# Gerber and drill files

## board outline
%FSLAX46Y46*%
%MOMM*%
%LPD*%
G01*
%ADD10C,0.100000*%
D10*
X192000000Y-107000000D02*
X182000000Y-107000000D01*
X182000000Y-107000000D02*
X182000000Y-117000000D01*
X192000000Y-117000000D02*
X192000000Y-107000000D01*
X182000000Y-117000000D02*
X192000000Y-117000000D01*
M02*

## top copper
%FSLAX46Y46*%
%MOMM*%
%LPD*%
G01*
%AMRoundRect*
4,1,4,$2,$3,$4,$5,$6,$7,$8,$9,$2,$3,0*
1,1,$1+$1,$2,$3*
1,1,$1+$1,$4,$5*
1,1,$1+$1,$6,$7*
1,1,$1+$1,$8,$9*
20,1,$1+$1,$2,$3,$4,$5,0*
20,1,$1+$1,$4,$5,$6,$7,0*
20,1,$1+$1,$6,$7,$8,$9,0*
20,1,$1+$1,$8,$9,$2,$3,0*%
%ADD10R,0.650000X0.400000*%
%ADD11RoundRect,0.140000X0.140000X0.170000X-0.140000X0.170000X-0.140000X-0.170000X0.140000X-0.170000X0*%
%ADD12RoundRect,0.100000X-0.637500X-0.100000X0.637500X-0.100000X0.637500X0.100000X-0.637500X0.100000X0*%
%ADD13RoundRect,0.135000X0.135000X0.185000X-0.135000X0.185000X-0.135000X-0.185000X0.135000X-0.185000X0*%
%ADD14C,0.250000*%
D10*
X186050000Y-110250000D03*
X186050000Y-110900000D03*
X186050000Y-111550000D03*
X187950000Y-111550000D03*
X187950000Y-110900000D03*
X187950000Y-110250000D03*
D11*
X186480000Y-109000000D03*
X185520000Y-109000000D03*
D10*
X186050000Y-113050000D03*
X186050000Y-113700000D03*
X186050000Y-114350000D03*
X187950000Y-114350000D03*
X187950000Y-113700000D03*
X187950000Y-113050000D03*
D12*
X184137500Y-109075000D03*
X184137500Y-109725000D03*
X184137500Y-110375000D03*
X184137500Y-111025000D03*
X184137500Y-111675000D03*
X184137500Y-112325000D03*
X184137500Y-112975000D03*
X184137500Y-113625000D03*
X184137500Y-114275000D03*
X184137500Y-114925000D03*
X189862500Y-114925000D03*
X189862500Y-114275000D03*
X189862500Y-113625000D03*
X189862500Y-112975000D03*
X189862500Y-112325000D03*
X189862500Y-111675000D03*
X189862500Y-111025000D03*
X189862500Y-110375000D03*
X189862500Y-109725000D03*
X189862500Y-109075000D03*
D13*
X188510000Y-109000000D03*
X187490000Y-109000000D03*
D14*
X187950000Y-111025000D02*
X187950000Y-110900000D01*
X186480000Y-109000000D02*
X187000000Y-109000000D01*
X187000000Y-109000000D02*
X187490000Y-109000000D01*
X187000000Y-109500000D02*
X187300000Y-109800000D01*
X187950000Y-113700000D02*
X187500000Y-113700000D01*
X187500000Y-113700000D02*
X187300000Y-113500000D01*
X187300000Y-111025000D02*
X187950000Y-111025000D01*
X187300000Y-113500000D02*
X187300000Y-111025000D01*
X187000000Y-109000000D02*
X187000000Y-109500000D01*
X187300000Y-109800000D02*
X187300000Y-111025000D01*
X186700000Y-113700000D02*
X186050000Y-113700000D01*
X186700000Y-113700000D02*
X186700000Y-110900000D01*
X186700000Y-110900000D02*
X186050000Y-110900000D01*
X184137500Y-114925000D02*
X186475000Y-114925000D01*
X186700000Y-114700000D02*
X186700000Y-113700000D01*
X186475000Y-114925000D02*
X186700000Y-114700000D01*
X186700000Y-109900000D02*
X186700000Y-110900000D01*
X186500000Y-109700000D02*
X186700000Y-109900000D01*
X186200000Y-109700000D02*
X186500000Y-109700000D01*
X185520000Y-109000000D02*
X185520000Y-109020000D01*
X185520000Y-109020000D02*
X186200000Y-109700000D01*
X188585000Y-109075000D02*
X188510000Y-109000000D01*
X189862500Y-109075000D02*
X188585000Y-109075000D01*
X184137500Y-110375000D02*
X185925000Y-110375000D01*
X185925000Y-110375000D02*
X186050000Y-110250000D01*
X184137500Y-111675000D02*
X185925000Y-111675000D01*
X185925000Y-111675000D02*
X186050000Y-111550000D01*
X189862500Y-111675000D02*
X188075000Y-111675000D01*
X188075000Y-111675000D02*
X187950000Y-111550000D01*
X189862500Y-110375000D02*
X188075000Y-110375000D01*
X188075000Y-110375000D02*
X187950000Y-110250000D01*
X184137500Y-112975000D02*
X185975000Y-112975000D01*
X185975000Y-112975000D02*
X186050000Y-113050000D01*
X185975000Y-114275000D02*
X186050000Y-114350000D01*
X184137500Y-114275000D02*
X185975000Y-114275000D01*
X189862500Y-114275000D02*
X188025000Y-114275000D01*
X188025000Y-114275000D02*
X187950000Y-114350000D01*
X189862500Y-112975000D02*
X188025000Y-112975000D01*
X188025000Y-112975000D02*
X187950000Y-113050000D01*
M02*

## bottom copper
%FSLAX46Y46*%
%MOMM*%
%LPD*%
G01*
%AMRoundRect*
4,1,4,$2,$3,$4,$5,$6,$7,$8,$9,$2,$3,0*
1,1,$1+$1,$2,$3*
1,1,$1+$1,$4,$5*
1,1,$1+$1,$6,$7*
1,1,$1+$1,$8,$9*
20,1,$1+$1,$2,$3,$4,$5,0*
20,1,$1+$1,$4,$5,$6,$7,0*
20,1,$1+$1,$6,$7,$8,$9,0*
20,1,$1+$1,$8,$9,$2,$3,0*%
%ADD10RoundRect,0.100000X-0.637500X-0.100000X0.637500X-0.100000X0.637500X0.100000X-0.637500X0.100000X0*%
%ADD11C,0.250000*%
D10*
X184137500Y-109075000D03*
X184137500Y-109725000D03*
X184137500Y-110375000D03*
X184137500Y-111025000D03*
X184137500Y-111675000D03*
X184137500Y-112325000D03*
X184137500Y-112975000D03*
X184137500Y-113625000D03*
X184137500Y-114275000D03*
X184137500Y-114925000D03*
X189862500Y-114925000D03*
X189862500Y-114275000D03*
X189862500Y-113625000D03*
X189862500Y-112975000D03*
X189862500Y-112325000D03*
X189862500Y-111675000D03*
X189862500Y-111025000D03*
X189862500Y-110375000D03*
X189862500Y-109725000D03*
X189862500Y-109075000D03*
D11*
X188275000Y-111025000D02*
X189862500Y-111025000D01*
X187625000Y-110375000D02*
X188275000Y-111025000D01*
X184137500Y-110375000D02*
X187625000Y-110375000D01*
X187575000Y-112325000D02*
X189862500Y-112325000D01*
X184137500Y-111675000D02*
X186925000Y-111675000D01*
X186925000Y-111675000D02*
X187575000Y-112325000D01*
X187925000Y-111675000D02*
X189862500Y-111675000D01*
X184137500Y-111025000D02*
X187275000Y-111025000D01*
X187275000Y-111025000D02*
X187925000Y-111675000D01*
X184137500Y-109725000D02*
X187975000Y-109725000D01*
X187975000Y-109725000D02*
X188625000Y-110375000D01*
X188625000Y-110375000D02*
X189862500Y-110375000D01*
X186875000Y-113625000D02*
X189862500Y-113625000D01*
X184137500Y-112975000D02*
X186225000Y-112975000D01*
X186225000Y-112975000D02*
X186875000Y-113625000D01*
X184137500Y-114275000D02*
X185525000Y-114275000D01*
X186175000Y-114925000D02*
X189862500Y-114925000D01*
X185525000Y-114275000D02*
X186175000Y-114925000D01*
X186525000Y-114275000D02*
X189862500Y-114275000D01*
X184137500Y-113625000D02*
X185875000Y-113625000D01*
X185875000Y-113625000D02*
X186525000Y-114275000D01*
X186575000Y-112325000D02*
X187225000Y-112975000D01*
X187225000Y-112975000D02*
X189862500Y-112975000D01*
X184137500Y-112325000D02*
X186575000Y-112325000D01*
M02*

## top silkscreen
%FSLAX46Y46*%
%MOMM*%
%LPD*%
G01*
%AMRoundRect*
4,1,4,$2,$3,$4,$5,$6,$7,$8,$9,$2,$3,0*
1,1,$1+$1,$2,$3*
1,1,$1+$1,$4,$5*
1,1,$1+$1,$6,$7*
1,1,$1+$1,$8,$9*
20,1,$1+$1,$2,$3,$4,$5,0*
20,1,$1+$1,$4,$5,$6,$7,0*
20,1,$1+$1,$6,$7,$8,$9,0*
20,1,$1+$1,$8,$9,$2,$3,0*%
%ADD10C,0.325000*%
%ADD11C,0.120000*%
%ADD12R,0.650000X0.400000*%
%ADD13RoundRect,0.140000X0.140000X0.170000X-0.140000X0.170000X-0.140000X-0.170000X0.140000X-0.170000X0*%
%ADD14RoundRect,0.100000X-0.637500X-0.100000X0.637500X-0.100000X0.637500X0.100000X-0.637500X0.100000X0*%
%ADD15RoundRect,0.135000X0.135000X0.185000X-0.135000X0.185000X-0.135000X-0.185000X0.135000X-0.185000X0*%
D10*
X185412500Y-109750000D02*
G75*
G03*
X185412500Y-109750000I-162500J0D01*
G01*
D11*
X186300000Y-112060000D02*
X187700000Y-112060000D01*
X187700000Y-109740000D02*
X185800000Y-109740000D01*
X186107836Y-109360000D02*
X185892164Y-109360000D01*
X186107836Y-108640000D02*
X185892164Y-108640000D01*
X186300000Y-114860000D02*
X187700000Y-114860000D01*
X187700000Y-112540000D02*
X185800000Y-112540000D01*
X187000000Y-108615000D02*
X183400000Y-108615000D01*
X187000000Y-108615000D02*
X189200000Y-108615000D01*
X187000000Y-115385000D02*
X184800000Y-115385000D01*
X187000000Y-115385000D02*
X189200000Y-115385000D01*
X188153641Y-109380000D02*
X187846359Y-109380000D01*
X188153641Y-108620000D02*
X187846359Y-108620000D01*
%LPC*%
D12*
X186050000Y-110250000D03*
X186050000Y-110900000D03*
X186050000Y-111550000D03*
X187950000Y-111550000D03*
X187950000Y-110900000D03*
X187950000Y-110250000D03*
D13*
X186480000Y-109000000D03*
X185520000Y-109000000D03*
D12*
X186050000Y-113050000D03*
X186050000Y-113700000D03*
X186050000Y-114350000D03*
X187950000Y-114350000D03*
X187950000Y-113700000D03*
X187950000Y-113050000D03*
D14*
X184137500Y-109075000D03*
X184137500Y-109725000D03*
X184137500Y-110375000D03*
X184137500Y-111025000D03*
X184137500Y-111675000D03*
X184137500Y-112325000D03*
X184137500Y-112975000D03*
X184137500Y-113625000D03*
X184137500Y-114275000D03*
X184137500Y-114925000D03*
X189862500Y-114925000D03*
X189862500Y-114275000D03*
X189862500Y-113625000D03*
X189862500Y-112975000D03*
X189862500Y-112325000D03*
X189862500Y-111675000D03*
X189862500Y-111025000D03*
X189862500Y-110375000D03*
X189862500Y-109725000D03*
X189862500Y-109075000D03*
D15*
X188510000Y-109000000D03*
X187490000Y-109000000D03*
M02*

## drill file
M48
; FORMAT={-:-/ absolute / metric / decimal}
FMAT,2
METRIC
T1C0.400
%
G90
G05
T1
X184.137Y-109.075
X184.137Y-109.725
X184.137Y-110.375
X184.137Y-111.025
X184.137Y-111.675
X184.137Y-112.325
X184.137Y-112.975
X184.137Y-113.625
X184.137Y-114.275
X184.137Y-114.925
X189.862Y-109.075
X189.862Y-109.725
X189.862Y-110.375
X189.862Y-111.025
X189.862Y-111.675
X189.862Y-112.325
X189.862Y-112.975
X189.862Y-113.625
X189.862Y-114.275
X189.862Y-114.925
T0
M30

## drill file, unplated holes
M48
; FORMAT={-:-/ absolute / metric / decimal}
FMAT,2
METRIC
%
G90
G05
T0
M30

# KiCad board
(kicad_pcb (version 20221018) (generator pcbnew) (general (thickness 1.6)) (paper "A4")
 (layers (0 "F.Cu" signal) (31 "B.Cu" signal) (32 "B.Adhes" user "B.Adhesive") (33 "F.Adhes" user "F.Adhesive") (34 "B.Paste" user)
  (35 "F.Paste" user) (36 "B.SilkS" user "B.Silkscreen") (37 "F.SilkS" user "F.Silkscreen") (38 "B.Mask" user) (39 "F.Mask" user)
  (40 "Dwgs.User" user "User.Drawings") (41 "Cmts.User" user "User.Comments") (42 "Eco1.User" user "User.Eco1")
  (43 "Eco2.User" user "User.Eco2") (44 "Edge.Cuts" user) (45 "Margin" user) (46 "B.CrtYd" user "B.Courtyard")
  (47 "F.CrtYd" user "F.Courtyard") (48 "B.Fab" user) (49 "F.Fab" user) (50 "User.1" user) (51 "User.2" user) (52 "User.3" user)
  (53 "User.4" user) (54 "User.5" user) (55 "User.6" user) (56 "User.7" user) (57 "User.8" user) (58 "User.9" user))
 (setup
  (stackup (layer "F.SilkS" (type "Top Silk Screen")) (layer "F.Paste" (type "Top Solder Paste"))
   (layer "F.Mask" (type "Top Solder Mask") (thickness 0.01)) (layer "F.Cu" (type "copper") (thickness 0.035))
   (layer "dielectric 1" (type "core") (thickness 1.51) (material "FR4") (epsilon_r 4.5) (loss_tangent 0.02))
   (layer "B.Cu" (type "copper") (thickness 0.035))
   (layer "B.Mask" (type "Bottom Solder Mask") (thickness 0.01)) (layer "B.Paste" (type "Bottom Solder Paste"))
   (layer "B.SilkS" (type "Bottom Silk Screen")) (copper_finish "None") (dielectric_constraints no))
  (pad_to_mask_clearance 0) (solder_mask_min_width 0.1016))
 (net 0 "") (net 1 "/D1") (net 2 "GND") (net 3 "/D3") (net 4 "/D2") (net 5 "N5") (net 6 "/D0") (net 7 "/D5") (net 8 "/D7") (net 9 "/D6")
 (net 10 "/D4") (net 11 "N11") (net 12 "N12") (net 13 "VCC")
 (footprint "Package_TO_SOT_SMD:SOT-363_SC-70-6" (layer "F.Cu") (at 187 110.9)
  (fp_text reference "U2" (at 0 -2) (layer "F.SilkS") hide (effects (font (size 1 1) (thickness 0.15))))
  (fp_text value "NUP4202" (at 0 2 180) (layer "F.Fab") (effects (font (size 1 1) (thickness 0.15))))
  (fp_line (start -0.7 1.16) (end 0.7 1.16) (stroke (width 0.12) (type solid)) (layer "F.SilkS"))
  (fp_line (start 0.7 -1.16) (end -1.2 -1.16) (stroke (width 0.12) (type solid)) (layer "F.SilkS"))
  (pad "1" smd rect (at -0.95 -0.65) (size 0.65 0.4) (layers "F.Cu" "F.Paste" "F.Mask") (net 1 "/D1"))
  (pad "2" smd rect (at -0.95 0) (size 0.65 0.4) (layers "F.Cu" "F.Paste" "F.Mask") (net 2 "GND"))
  (pad "3" smd rect (at -0.95 0.65) (size 0.65 0.4) (layers "F.Cu" "F.Paste" "F.Mask") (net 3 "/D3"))
  (pad "4" smd rect (at 0.95 0.65) (size 0.65 0.4) (layers "F.Cu" "F.Paste" "F.Mask") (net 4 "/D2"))
  (pad "5" smd rect (at 0.95 0) (size 0.65 0.4) (layers "F.Cu" "F.Paste" "F.Mask") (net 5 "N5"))
  (pad "6" smd rect (at 0.95 -0.65) (size 0.65 0.4) (layers "F.Cu" "F.Paste" "F.Mask") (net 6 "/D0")))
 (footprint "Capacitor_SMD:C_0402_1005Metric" (layer "F.Cu") (at 186 109 180)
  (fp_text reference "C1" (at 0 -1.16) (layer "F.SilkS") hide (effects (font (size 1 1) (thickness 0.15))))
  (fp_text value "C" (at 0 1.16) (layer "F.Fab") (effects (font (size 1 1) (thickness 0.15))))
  (fp_line (start -0.107836 -0.36) (end 0.107836 -0.36) (stroke (width 0.12) (type solid)) (layer "F.SilkS"))
  (fp_line (start -0.107836 0.36) (end 0.107836 0.36) (stroke (width 0.12) (type solid)) (layer "F.SilkS"))
  (pad "1" smd roundrect (at -0.48 0 180) (size 0.56 0.62) (layers "F.Cu" "F.Paste" "F.Mask") (roundrect_rratio 0.25) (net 5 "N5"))
  (pad "2" smd roundrect (at 0.48 0 180) (size 0.56 0.62) (layers "F.Cu" "F.Paste" "F.Mask") (roundrect_rratio 0.25) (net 2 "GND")))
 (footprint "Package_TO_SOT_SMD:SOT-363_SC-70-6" (layer "F.Cu") (at 187 113.7)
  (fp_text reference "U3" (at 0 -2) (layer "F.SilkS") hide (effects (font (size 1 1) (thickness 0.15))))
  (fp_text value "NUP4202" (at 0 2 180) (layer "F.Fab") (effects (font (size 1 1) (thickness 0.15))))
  (fp_line (start -0.7 1.16) (end 0.7 1.16) (stroke (width 0.12) (type solid)) (layer "F.SilkS"))
  (fp_line (start 0.7 -1.16) (end -1.2 -1.16) (stroke (width 0.12) (type solid)) (layer "F.SilkS"))
  (pad "1" smd rect (at -0.95 -0.65) (size 0.65 0.4) (layers "F.Cu" "F.Paste" "F.Mask") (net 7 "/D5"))
  (pad "2" smd rect (at -0.95 0) (size 0.65 0.4) (layers "F.Cu" "F.Paste" "F.Mask") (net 2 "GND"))
  (pad "3" smd rect (at -0.95 0.65) (size 0.65 0.4) (layers "F.Cu" "F.Paste" "F.Mask") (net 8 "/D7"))
  (pad "4" smd rect (at 0.95 0.65) (size 0.65 0.4) (layers "F.Cu" "F.Paste" "F.Mask") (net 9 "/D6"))
  (pad "5" smd rect (at 0.95 0) (size 0.65 0.4) (layers "F.Cu" "F.Paste" "F.Mask") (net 5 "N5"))
  (pad "6" smd rect (at 0.95 -0.65) (size 0.65 0.4) (layers "F.Cu" "F.Paste" "F.Mask") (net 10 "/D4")))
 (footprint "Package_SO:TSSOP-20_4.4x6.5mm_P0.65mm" (layer "F.Cu") (at 187 112)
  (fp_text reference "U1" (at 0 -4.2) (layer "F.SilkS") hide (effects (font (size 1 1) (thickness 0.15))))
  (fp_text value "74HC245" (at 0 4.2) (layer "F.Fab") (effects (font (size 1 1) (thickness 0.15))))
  (fp_line (start 0 -3.385) (end -3.6 -3.385) (stroke (width 0.12) (type solid)) (layer "F.SilkS"))
  (fp_line (start 0 -3.385) (end 2.2 -3.385) (stroke (width 0.12) (type solid)) (layer "F.SilkS"))
  (fp_line (start 0 3.385) (end -2.2 3.385) (stroke (width 0.12) (type solid)) (layer "F.SilkS"))
  (fp_line (start 0 3.385) (end 2.2 3.385) (stroke (width 0.12) (type solid)) (layer "F.SilkS"))
  (pad "1" thru_hole roundrect (at -2.8625 -2.925) (size 1.475 0.4) (drill 0.4) (layers "*.Cu" "*.Mask") (roundrect_rratio 0.25)
   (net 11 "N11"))
  (pad "2" thru_hole roundrect (at -2.8625 -2.275) (size 1.475 0.4) (drill 0.4) (layers "*.Cu" "*.Mask") (roundrect_rratio 0.25)
   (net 6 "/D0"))
  (pad "3" thru_hole roundrect (at -2.8625 -1.625) (size 1.475 0.4) (drill 0.4) (layers "*.Cu" "*.Mask") (roundrect_rratio 0.25)
   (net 1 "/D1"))
  (pad "4" thru_hole roundrect (at -2.8625 -0.975) (size 1.475 0.4) (drill 0.4) (layers "*.Cu" "*.Mask") (roundrect_rratio 0.25)
   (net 4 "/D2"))
  (pad "5" thru_hole roundrect (at -2.8625 -0.325) (size 1.475 0.4) (drill 0.4) (layers "*.Cu" "*.Mask") (roundrect_rratio 0.25)
   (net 3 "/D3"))
  (pad "6" thru_hole roundrect (at -2.8625 0.325) (size 1.475 0.4) (drill 0.4) (layers "*.Cu" "*.Mask") (roundrect_rratio 0.25)
   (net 10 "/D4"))
  (pad "7" thru_hole roundrect (at -2.8625 0.975) (size 1.475 0.4) (drill 0.4) (layers "*.Cu" "*.Mask") (roundrect_rratio 0.25)
   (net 7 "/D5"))
  (pad "8" thru_hole roundrect (at -2.8625 1.625) (size 1.475 0.4) (drill 0.4) (layers "*.Cu" "*.Mask") (roundrect_rratio 0.25)
   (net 9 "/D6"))
  (pad "9" thru_hole roundrect (at -2.8625 2.275) (size 1.475 0.4) (drill 0.4) (layers "*.Cu" "*.Mask") (roundrect_rratio 0.25)
   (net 8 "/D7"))
  (pad "10" thru_hole roundrect (at -2.8625 2.925) (size 1.475 0.4) (drill 0.4) (layers "*.Cu" "*.Mask") (roundrect_rratio 0.25)
   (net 2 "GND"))
  (pad "11" thru_hole roundrect (at 2.8625 2.925) (size 1.475 0.4) (drill 0.4) (layers "*.Cu" "*.Mask") (roundrect_rratio 0.25)
   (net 8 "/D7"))
  (pad "12" thru_hole roundrect (at 2.8625 2.275) (size 1.475 0.4) (drill 0.4) (layers "*.Cu" "*.Mask") (roundrect_rratio 0.25)
   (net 9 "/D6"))
  (pad "13" thru_hole roundrect (at 2.8625 1.625) (size 1.475 0.4) (drill 0.4) (layers "*.Cu" "*.Mask") (roundrect_rratio 0.25)
   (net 7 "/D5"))
  (pad "14" thru_hole roundrect (at 2.8625 0.975) (size 1.475 0.4) (drill 0.4) (layers "*.Cu" "*.Mask") (roundrect_rratio 0.25)
   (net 10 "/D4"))
  (pad "15" thru_hole roundrect (at 2.8625 0.325) (size 1.475 0.4) (drill 0.4) (layers "*.Cu" "*.Mask") (roundrect_rratio 0.25)
   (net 3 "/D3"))
  (pad "16" thru_hole roundrect (at 2.8625 -0.325) (size 1.475 0.4) (drill 0.4) (layers "*.Cu" "*.Mask") (roundrect_rratio 0.25)
   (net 4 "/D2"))
  (pad "17" thru_hole roundrect (at 2.8625 -0.975) (size 1.475 0.4) (drill 0.4) (layers "*.Cu" "*.Mask") (roundrect_rratio 0.25)
   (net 1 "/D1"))
  (pad "18" thru_hole roundrect (at 2.8625 -1.625) (size 1.475 0.4) (drill 0.4) (layers "*.Cu" "*.Mask") (roundrect_rratio 0.25)
   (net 6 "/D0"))
  (pad "19" thru_hole roundrect (at 2.8625 -2.275) (size 1.475 0.4) (drill 0.4) (layers "*.Cu" "*.Mask") (roundrect_rratio 0.25)
   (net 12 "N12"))
  (pad "20" thru_hole roundrect (at 2.8625 -2.925) (size 1.475 0.4) (drill 0.4) (layers "*.Cu" "*.Mask") (roundrect_rratio 0.25)
   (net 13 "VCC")))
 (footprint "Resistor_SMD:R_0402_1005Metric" (layer "F.Cu") (at 188 109 180)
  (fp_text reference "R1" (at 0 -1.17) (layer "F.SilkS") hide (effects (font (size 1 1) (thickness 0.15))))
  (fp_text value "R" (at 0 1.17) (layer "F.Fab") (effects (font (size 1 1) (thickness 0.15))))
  (fp_line (start -0.153641 -0.38) (end 0.153641 -0.38) (stroke (width 0.12) (type solid)) (layer "F.SilkS"))
  (fp_line (start -0.153641 0.38) (end 0.153641 0.38) (stroke (width 0.12) (type solid)) (layer "F.SilkS"))
  (pad "1" smd roundrect (at -0.51 0 180) (size 0.54 0.64) (layers "F.Cu" "F.Paste" "F.Mask") (roundrect_rratio 0.25) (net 13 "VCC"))
  (pad "2" smd roundrect (at 0.51 0 180) (size 0.54 0.64) (layers "F.Cu" "F.Paste" "F.Mask") (roundrect_rratio 0.25) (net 5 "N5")))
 (gr_circle (center 185.25 109.75) (end 185.5 109.75) (stroke (width 0.15) (type solid)) (fill solid) (layer "F.SilkS"))
 (gr_line (start 192 107) (end 182 107) (stroke (width 0.1) (type solid)) (layer "Edge.Cuts"))
 (gr_line (start 182 107) (end 182 117) (stroke (width 0.1) (type solid)) (layer "Edge.Cuts"))
 (gr_line (start 192 117) (end 192 107) (stroke (width 0.1) (type solid)) (layer "Edge.Cuts"))
 (gr_line (start 182 117) (end 192 117) (stroke (width 0.1) (type solid)) (layer "Edge.Cuts"))
 (segment (start 187.95 111.025) (end 187.95 110.9) (width 0.25) (layer "F.Cu") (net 5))
 (segment (start 186.48 109) (end 187 109) (width 0.25) (layer "F.Cu") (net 5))
 (segment (start 187 109) (end 187.49 109) (width 0.25) (layer "F.Cu") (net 5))
 (segment (start 187 109.5) (end 187.3 109.8) (width 0.25) (layer "F.Cu") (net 5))
 (segment (start 187.95 113.7) (end 187.5 113.7) (width 0.25) (layer "F.Cu") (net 5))
 (segment (start 187.5 113.7) (end 187.3 113.5) (width 0.25) (layer "F.Cu") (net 5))
 (segment (start 187.3 111.025) (end 187.95 111.025) (width 0.25) (layer "F.Cu") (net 5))
 (segment (start 187.3 113.5) (end 187.3 111.025) (width 0.25) (layer "F.Cu") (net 5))
 (segment (start 187 109) (end 187 109.5) (width 0.25) (layer "F.Cu") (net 5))
 (segment (start 187.3 109.8) (end 187.3 111.025) (width 0.25) (layer "F.Cu") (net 5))
 (segment (start 186.7 113.7) (end 186.05 113.7) (width 0.25) (layer "F.Cu") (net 2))
 (segment (start 186.7 113.7) (end 186.7 110.9) (width 0.25) (layer "F.Cu") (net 2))
 (segment (start 186.7 110.9) (end 186.05 110.9) (width 0.25) (layer "F.Cu") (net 2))
 (segment (start 184.1375 114.925) (end 186.475 114.925) (width 0.25) (layer "F.Cu") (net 2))
 (segment (start 186.7 114.7) (end 186.7 113.7) (width 0.25) (layer "F.Cu") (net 2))
 (segment (start 186.475 114.925) (end 186.7 114.7) (width 0.25) (layer "F.Cu") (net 2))
 (segment (start 186.7 109.9) (end 186.7 110.9) (width 0.25) (layer "F.Cu") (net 2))
 (segment (start 186.5 109.7) (end 186.7 109.9) (width 0.25) (layer "F.Cu") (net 2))
 (segment (start 186.2 109.7) (end 186.5 109.7) (width 0.25) (layer "F.Cu") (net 2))
 (segment (start 185.52 109) (end 185.52 109.02) (width 0.25) (layer "F.Cu") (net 2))
 (segment (start 185.52 109.02) (end 186.2 109.7) (width 0.25) (layer "F.Cu") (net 2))
 (segment (start 188.585 109.075) (end 188.51 109) (width 0.25) (layer "F.Cu") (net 13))
 (segment (start 189.8625 109.075) (end 188.585 109.075) (width 0.25) (layer "F.Cu") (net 13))
 (segment (start 184.1375 110.375) (end 185.925 110.375) (width 0.25) (layer "F.Cu") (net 1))
 (segment (start 185.925 110.375) (end 186.05 110.25) (width 0.25) (layer "F.Cu") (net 1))
 (segment (start 188.275 111.025) (end 189.8625 111.025) (width 0.25) (layer "B.Cu") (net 1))
 (segment (start 187.625 110.375) (end 188.275 111.025) (width 0.25) (layer "B.Cu") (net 1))
 (segment (start 184.1375 110.375) (end 187.625 110.375) (width 0.25) (layer "B.Cu") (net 1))
 (segment (start 184.1375 111.675) (end 185.925 111.675) (width 0.25) (layer "F.Cu") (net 3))
 (segment (start 185.925 111.675) (end 186.05 111.55) (width 0.25) (layer "F.Cu") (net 3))
 (segment (start 187.575 112.325) (end 189.8625 112.325) (width 0.25) (layer "B.Cu") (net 3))
 (segment (start 184.1375 111.675) (end 186.925 111.675) (width 0.25) (layer "B.Cu") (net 3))
 (segment (start 186.925 111.675) (end 187.575 112.325) (width 0.25) (layer "B.Cu") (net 3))
 (segment (start 189.8625 111.675) (end 188.075 111.675) (width 0.25) (layer "F.Cu") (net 4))
 (segment (start 188.075 111.675) (end 187.95 111.55) (width 0.25) (layer "F.Cu") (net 4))
 (segment (start 187.925 111.675) (end 189.8625 111.675) (width 0.25) (layer "B.Cu") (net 4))
 (segment (start 184.1375 111.025) (end 187.275 111.025) (width 0.25) (layer "B.Cu") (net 4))
 (segment (start 187.275 111.025) (end 187.925 111.675) (width 0.25) (layer "B.Cu") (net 4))
 (segment (start 189.8625 110.375) (end 188.075 110.375) (width 0.25) (layer "F.Cu") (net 6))
 (segment (start 188.075 110.375) (end 187.95 110.25) (width 0.25) (layer "F.Cu") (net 6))
 (segment (start 184.1375 109.725) (end 187.975 109.725) (width 0.25) (layer "B.Cu") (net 6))
 (segment (start 187.975 109.725) (end 188.625 110.375) (width 0.25) (layer "B.Cu") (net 6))
 (segment (start 188.625 110.375) (end 189.8625 110.375) (width 0.25) (layer "B.Cu") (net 6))
 (segment (start 184.1375 112.975) (end 185.975 112.975) (width 0.25) (layer "F.Cu") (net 7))
 (segment (start 185.975 112.975) (end 186.05 113.05) (width 0.25) (layer "F.Cu") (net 7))
 (segment (start 186.875 113.625) (end 189.8625 113.625) (width 0.25) (layer "B.Cu") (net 7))
 (segment (start 184.1375 112.975) (end 186.225 112.975) (width 0.25) (layer "B.Cu") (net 7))
 (segment (start 186.225 112.975) (end 186.875 113.625) (width 0.25) (layer "B.Cu") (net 7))
 (segment (start 185.975 114.275) (end 186.05 114.35) (width 0.25) (layer "F.Cu") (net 8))
 (segment (start 184.1375 114.275) (end 185.975 114.275) (width 0.25) (layer "F.Cu") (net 8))
 (segment (start 184.1375 114.275) (end 185.525 114.275) (width 0.25) (layer "B.Cu") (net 8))
 (segment (start 186.175 114.925) (end 189.8625 114.925) (width 0.25) (layer "B.Cu") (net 8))
 (segment (start 185.525 114.275) (end 186.175 114.925) (width 0.25) (layer "B.Cu") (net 8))
 (segment (start 189.8625 114.275) (end 188.025 114.275) (width 0.25) (layer "F.Cu") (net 9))
 (segment (start 188.025 114.275) (end 187.95 114.35) (width 0.25) (layer "F.Cu") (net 9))
 (segment (start 186.525 114.275) (end 189.8625 114.275) (width 0.25) (layer "B.Cu") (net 9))
 (segment (start 184.1375 113.625) (end 185.875 113.625) (width 0.25) (layer "B.Cu") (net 9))
 (segment (start 185.875 113.625) (end 186.525 114.275) (width 0.25) (layer "B.Cu") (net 9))
 (segment (start 189.8625 112.975) (end 188.025 112.975) (width 0.25) (layer "F.Cu") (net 10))
 (segment (start 188.025 112.975) (end 187.95 113.05) (width 0.25) (layer "F.Cu") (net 10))
 (segment (start 186.575 112.325) (end 187.225 112.975) (width 0.25) (layer "B.Cu") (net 10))
 (segment (start 187.225 112.975) (end 189.8625 112.975) (width 0.25) (layer "B.Cu") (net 10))
 (segment (start 184.1375 112.325) (end 186.575 112.325) (width 0.25) (layer "B.Cu") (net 10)))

